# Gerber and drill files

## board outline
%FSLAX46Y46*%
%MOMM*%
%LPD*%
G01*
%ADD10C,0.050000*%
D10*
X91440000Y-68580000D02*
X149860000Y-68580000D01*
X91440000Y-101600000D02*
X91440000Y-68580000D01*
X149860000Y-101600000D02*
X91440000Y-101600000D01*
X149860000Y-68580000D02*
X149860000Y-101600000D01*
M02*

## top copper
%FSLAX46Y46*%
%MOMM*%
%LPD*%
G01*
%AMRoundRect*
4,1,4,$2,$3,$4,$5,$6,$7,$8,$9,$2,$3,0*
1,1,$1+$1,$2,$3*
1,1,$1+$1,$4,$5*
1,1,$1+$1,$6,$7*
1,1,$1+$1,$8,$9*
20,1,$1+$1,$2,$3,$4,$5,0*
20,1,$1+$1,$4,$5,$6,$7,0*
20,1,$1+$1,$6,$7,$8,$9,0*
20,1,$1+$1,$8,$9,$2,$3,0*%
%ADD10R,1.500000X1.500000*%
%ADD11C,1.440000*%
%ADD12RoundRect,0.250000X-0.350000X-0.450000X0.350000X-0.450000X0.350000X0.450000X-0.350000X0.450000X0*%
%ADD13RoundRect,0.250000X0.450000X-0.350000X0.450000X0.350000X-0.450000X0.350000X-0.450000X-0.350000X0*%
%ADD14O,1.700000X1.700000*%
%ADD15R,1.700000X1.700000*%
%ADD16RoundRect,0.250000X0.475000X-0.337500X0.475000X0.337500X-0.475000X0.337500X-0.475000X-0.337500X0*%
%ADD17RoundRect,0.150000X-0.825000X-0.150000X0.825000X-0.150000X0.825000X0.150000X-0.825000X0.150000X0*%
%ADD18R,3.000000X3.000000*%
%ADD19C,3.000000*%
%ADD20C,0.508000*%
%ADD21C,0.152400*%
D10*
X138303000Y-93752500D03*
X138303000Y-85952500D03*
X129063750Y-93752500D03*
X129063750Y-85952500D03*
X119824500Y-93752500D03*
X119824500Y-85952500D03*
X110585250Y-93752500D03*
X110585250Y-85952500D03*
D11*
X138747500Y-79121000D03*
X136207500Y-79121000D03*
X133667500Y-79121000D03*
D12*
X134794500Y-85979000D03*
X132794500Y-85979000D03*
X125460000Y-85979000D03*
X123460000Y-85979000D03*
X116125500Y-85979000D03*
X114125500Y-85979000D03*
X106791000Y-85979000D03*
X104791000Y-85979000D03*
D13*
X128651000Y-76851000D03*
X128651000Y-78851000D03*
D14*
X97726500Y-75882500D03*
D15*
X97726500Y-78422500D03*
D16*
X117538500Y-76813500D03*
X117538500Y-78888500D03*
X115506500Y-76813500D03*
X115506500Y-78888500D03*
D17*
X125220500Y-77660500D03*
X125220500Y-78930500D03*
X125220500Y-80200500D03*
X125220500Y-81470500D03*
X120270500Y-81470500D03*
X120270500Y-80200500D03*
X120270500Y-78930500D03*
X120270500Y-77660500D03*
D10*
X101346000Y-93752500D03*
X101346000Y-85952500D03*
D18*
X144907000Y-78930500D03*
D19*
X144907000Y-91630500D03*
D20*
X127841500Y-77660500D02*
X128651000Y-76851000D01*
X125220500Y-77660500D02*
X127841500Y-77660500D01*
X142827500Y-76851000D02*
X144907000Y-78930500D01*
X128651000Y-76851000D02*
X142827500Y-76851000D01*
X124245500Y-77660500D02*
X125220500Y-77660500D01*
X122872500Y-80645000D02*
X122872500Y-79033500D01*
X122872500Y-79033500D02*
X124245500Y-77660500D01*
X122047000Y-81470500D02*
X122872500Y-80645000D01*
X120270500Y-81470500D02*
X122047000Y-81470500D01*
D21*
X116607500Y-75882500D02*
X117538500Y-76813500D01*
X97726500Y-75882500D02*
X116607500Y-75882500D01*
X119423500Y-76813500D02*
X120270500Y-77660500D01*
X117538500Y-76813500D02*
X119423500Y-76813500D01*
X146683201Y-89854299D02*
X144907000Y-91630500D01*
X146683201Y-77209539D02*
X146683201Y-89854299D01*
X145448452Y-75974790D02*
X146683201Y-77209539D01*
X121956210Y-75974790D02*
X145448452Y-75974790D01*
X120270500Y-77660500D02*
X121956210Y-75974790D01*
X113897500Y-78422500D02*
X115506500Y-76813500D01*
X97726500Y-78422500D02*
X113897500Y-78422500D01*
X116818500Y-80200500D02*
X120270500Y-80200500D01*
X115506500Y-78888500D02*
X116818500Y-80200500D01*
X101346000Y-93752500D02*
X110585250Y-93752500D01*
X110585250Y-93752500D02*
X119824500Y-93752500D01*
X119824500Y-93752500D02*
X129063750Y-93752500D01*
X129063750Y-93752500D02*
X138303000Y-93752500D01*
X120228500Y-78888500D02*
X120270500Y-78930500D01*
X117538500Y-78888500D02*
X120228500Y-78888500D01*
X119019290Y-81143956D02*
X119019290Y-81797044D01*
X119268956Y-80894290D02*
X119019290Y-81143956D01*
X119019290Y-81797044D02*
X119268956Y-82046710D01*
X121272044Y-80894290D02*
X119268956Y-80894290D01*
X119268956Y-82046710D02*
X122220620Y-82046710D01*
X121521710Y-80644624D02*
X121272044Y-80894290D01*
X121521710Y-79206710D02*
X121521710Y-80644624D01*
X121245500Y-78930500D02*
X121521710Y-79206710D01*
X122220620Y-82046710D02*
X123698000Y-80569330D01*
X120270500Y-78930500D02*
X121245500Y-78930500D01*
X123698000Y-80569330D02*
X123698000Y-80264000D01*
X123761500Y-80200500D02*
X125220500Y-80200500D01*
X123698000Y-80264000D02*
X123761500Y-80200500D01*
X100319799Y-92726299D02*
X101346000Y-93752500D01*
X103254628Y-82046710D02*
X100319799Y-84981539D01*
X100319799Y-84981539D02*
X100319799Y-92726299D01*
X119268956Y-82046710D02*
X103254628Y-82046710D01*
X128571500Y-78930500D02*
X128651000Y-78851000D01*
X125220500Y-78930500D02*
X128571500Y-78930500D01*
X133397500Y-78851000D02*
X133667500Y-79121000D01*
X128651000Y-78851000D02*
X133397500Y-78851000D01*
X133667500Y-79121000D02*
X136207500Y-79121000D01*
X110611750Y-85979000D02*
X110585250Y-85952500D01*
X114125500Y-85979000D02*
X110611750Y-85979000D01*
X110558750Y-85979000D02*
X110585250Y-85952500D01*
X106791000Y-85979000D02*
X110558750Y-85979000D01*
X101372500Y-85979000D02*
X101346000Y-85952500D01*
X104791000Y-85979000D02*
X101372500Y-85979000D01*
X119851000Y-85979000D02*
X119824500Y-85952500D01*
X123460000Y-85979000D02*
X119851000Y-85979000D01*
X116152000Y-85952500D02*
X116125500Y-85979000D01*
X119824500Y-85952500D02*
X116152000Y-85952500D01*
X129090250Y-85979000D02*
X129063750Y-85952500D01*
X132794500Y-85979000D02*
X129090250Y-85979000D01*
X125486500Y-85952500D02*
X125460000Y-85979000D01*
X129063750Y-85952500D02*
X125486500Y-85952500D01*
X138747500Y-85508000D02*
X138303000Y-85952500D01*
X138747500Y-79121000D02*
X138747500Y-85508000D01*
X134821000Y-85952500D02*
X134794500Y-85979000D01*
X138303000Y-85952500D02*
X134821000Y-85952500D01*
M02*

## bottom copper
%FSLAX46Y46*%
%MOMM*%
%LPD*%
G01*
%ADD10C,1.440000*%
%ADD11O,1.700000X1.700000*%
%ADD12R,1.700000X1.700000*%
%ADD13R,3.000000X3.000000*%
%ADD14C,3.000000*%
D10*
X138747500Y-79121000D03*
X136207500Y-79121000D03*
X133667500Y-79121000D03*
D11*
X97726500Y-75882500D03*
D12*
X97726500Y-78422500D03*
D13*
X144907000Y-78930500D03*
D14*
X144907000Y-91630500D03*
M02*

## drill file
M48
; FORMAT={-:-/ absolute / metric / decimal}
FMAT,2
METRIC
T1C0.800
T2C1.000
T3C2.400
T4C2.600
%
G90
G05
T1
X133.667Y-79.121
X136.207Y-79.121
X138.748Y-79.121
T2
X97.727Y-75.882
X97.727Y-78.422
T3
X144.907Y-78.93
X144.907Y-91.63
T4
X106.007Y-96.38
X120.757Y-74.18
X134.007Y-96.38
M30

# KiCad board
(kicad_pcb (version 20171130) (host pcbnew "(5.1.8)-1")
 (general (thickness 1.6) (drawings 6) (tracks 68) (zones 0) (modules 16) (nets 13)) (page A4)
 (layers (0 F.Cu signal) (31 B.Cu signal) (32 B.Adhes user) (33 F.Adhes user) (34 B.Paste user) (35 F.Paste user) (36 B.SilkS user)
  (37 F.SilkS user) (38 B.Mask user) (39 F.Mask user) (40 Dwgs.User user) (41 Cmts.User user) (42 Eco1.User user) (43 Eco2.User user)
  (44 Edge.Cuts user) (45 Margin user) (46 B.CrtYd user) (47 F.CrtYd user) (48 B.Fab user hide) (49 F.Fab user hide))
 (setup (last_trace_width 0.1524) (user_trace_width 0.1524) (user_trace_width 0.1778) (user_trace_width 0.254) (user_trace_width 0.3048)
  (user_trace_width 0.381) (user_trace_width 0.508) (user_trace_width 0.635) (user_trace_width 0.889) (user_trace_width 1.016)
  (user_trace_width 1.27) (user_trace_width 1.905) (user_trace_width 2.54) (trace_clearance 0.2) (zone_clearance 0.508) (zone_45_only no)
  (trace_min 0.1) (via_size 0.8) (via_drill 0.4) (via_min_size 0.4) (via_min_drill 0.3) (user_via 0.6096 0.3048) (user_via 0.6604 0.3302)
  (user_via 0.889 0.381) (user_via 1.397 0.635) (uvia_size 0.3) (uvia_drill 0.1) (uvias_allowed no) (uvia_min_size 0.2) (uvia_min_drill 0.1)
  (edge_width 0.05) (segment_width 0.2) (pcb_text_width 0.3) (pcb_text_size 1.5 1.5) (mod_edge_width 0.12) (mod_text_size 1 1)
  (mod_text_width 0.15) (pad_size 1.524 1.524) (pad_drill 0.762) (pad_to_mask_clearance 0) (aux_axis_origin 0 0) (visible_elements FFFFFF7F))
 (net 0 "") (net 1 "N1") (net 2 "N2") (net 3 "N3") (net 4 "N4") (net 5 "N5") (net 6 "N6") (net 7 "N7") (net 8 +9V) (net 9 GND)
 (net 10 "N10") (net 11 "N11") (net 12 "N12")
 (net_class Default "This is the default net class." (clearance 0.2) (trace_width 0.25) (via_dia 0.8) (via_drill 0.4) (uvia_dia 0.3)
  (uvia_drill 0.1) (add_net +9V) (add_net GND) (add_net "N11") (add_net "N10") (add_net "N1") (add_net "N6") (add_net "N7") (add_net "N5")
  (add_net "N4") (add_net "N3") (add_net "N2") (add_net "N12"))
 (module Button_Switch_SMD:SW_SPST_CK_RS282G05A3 (layer F.Cu) (at 138.303 89.8525 270)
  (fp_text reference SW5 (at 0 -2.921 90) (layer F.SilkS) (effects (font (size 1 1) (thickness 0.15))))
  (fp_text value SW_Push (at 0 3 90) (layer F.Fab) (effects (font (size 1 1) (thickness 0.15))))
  (pad 2 smd rect (at 3.9 0 270) (size 1.5 1.5) (layers F.Cu F.Paste F.Mask) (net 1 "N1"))
  (pad 1 smd rect (at -3.9 0 270) (size 1.5 1.5) (layers F.Cu F.Paste F.Mask) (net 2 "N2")))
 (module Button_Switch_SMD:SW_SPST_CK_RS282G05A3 (layer F.Cu) (at 129.06375 89.8525 270)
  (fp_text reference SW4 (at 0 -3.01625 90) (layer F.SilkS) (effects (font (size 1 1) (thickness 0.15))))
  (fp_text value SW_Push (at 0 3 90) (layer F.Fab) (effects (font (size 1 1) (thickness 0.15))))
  (pad 2 smd rect (at 3.9 0 270) (size 1.5 1.5) (layers F.Cu F.Paste F.Mask) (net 1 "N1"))
  (pad 1 smd rect (at -3.9 0 270) (size 1.5 1.5) (layers F.Cu F.Paste F.Mask) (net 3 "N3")))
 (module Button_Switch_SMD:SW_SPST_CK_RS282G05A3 (layer F.Cu) (at 119.8245 89.8525 270)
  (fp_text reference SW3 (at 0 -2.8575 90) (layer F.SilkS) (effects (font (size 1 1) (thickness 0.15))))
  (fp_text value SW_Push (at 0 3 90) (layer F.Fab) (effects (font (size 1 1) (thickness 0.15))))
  (pad 2 smd rect (at 3.9 0 270) (size 1.5 1.5) (layers F.Cu F.Paste F.Mask) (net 1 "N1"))
  (pad 1 smd rect (at -3.9 0 270) (size 1.5 1.5) (layers F.Cu F.Paste F.Mask) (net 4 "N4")))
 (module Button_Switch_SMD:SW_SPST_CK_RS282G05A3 (layer F.Cu) (at 110.58525 89.8525 270)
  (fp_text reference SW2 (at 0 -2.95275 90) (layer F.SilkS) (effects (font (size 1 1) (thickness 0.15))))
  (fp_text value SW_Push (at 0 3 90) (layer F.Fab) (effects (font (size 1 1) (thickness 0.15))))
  (pad 2 smd rect (at 3.9 0 270) (size 1.5 1.5) (layers F.Cu F.Paste F.Mask) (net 1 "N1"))
  (pad 1 smd rect (at -3.9 0 270) (size 1.5 1.5) (layers F.Cu F.Paste F.Mask) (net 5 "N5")))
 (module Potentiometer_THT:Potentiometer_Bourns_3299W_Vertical (layer F.Cu) (at 133.6675 79.121 180)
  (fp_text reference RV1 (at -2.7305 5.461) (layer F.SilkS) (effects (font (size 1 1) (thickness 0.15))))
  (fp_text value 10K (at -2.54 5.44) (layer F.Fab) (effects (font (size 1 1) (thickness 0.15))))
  (pad 3 thru_hole circle (at -5.08 0 180) (size 1.44 1.44) (drill 0.8) (layers *.Cu *.Mask) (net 2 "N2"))
  (pad 2 thru_hole circle (at -2.54 0 180) (size 1.44 1.44) (drill 0.8) (layers *.Cu *.Mask) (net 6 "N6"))
  (pad 1 thru_hole circle (at 0 0 180) (size 1.44 1.44) (drill 0.8) (layers *.Cu *.Mask) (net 6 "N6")))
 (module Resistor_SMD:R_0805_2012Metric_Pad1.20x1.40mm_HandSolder (layer F.Cu) (at 133.7945 85.979)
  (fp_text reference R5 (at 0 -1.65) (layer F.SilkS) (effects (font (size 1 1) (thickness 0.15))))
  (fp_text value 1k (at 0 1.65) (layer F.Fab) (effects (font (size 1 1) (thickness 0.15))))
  (pad 2 smd roundrect (at 1 0) (size 1.2 1.4) (layers F.Cu F.Paste F.Mask) (roundrect_rratio 0.208333) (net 2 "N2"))
  (pad 1 smd roundrect (at -1 0) (size 1.2 1.4) (layers F.Cu F.Paste F.Mask) (roundrect_rratio 0.208333) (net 3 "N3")))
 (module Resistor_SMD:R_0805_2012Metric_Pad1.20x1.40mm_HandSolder (layer F.Cu) (at 124.46 85.979)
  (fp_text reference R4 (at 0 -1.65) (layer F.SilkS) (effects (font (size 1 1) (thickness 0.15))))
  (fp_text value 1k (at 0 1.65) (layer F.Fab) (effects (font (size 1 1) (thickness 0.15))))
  (pad 2 smd roundrect (at 1 0) (size 1.2 1.4) (layers F.Cu F.Paste F.Mask) (roundrect_rratio 0.208333) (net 3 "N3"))
  (pad 1 smd roundrect (at -1 0) (size 1.2 1.4) (layers F.Cu F.Paste F.Mask) (roundrect_rratio 0.208333) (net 4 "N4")))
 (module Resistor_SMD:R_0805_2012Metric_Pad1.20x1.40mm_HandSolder (layer F.Cu) (at 115.1255 85.979)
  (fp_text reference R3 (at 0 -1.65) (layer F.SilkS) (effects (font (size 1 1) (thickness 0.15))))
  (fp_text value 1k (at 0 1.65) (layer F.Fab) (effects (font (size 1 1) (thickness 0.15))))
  (pad 2 smd roundrect (at 1 0) (size 1.2 1.4) (layers F.Cu F.Paste F.Mask) (roundrect_rratio 0.208333) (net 4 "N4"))
  (pad 1 smd roundrect (at -1 0) (size 1.2 1.4) (layers F.Cu F.Paste F.Mask) (roundrect_rratio 0.208333) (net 5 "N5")))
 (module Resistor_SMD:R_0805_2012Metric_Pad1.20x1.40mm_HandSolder (layer F.Cu) (at 105.791 85.979)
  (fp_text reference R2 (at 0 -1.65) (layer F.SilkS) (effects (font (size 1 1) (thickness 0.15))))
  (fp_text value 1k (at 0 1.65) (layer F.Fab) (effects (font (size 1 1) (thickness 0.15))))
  (pad 2 smd roundrect (at 1 0) (size 1.2 1.4) (layers F.Cu F.Paste F.Mask) (roundrect_rratio 0.208333) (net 5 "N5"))
  (pad 1 smd roundrect (at -1 0) (size 1.2 1.4) (layers F.Cu F.Paste F.Mask) (roundrect_rratio 0.208333) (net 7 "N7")))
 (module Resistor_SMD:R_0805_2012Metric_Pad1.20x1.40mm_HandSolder (layer F.Cu) (at 128.651 77.851 90)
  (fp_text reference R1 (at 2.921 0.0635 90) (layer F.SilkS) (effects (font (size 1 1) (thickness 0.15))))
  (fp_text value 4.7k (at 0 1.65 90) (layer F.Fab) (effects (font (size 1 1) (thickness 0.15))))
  (pad 2 smd roundrect (at 1 0 90) (size 1.2 1.4) (layers F.Cu F.Paste F.Mask) (roundrect_rratio 0.208333) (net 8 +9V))
  (pad 1 smd roundrect (at -1 0 90) (size 1.2 1.4) (layers F.Cu F.Paste F.Mask) (roundrect_rratio 0.208333) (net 6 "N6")))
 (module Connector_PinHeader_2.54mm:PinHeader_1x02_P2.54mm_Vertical (layer F.Cu) (at 97.7265 78.4225 180)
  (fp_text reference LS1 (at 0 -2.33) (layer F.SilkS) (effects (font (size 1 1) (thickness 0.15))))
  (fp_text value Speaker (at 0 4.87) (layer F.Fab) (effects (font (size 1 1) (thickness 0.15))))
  (pad 2 thru_hole oval (at 0 2.54 180) (size 1.7 1.7) (drill 1) (layers *.Cu *.Mask) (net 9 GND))
  (pad 1 thru_hole rect (at 0 0 180) (size 1.7 1.7) (drill 1) (layers *.Cu *.Mask) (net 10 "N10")))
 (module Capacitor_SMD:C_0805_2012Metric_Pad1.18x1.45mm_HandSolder (layer F.Cu) (at 117.5385 77.851 90)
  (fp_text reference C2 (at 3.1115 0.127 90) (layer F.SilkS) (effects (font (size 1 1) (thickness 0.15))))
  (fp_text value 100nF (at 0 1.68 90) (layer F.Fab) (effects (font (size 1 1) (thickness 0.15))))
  (pad 2 smd roundrect (at 1.0375 0 90) (size 1.175 1.45) (layers F.Cu F.Paste F.Mask) (roundrect_rratio 0.212766) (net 9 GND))
  (pad 1 smd roundrect (at -1.0375 0 90) (size 1.175 1.45) (layers F.Cu F.Paste F.Mask) (roundrect_rratio 0.212766) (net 1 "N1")))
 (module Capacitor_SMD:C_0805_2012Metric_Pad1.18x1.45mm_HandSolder (layer F.Cu) (at 115.5065 77.851 90)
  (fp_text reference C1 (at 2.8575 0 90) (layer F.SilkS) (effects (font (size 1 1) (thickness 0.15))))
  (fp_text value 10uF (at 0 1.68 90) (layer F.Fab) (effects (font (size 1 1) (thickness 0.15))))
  (pad 2 smd roundrect (at 1.0375 0 90) (size 1.175 1.45) (layers F.Cu F.Paste F.Mask) (roundrect_rratio 0.212766) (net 10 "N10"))
  (pad 1 smd roundrect (at -1.0375 0 90) (size 1.175 1.45) (layers F.Cu F.Paste F.Mask) (roundrect_rratio 0.212766) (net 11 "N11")))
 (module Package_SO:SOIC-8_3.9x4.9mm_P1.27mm (layer F.Cu) (at 122.7455 79.5655)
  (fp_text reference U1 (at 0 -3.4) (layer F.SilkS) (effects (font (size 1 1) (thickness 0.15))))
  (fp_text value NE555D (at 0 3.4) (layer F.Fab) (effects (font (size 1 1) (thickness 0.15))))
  (pad 8 smd roundrect (at 2.475 -1.905) (size 1.95 0.6) (layers F.Cu F.Paste F.Mask) (roundrect_rratio 0.25) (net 8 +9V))
  (pad 7 smd roundrect (at 2.475 -0.635) (size 1.95 0.6) (layers F.Cu F.Paste F.Mask) (roundrect_rratio 0.25) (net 6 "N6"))
  (pad 6 smd roundrect (at 2.475 0.635) (size 1.95 0.6) (layers F.Cu F.Paste F.Mask) (roundrect_rratio 0.25) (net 1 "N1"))
  (pad 5 smd roundrect (at 2.475 1.905) (size 1.95 0.6) (layers F.Cu F.Paste F.Mask) (roundrect_rratio 0.25) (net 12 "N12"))
  (pad 4 smd roundrect (at -2.475 1.905) (size 1.95 0.6) (layers F.Cu F.Paste F.Mask) (roundrect_rratio 0.25) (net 8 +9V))
  (pad 3 smd roundrect (at -2.475 0.635) (size 1.95 0.6) (layers F.Cu F.Paste F.Mask) (roundrect_rratio 0.25) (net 11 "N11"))
  (pad 2 smd roundrect (at -2.475 -0.635) (size 1.95 0.6) (layers F.Cu F.Paste F.Mask) (roundrect_rratio 0.25) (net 1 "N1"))
  (pad 1 smd roundrect (at -2.475 -1.905) (size 1.95 0.6) (layers F.Cu F.Paste F.Mask) (roundrect_rratio 0.25) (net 9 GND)))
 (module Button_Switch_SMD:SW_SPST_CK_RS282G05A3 (layer F.Cu) (at 101.346 89.8525 270)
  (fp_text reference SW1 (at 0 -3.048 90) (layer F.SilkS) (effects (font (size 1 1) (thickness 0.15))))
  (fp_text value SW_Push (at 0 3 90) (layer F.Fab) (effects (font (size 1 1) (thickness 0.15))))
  (pad 2 smd rect (at 3.9 0 270) (size 1.5 1.5) (layers F.Cu F.Paste F.Mask) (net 1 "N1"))
  (pad 1 smd rect (at -3.9 0 270) (size 1.5 1.5) (layers F.Cu F.Paste F.Mask) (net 7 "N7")))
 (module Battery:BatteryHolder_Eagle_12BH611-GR (layer B.Cu) (at 144.907 78.9305)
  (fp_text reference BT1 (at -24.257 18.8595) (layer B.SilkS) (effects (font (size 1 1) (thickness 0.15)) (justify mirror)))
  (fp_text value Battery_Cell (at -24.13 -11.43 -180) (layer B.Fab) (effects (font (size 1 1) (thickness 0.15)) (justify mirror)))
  (pad "" np_thru_hole circle (at -24.15 -4.75) (size 2.6 2.6) (drill 2.6) (layers *.Cu *.Mask))
  (pad "" np_thru_hole circle (at -38.9 17.45) (size 2.6 2.6) (drill 2.6) (layers *.Cu *.Mask))
  (pad "" np_thru_hole circle (at -10.9 17.45) (size 2.6 2.6) (drill 2.6) (layers *.Cu *.Mask))
  (pad 1 thru_hole rect (at 0 0) (size 3 3) (drill 2.4) (layers *.Cu *.Mask) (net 8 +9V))
  (pad 2 thru_hole circle (at 0 12.7) (size 3 3) (drill 2.4) (layers *.Cu *.Mask) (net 9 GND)))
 (gr_line (start 91.44 68.58) (end 149.86 68.58) (layer Edge.Cuts) (width 0.05))
 (gr_line (start 91.44 101.6) (end 91.44 68.58) (layer Edge.Cuts) (width 0.05))
 (gr_line (start 149.86 101.6) (end 91.44 101.6) (layer Edge.Cuts) (width 0.05))
 (gr_line (start 149.86 68.58) (end 149.86 101.6) (layer Edge.Cuts) (width 0.05))
 (segment (start 127.8415 77.6605) (end 128.651 76.851) (width 0.508) (layer F.Cu) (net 8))
 (segment (start 125.2205 77.6605) (end 127.8415 77.6605) (width 0.508) (layer F.Cu) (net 8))
 (segment (start 142.8275 76.851) (end 144.907 78.9305) (width 0.508) (layer F.Cu) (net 8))
 (segment (start 128.651 76.851) (end 142.8275 76.851) (width 0.508) (layer F.Cu) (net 8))
 (segment (start 124.2455 77.6605) (end 125.2205 77.6605) (width 0.508) (layer F.Cu) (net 8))
 (segment (start 122.8725 80.645) (end 122.8725 79.0335) (width 0.508) (layer F.Cu) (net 8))
 (segment (start 122.8725 79.0335) (end 124.2455 77.6605) (width 0.508) (layer F.Cu) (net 8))
 (segment (start 122.047 81.4705) (end 122.8725 80.645) (width 0.508) (layer F.Cu) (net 8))
 (segment (start 120.2705 81.4705) (end 122.047 81.4705) (width 0.508) (layer F.Cu) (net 8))
 (segment (start 116.6075 75.8825) (end 117.5385 76.8135) (width 0.1524) (layer F.Cu) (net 9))
 (segment (start 97.7265 75.8825) (end 116.6075 75.8825) (width 0.1524) (layer F.Cu) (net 9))
 (segment (start 119.4235 76.8135) (end 120.2705 77.6605) (width 0.1524) (layer F.Cu) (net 9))
 (segment (start 117.5385 76.8135) (end 119.4235 76.8135) (width 0.1524) (layer F.Cu) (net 9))
 (segment (start 146.683201 89.854299) (end 144.907 91.6305) (width 0.1524) (layer F.Cu) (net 9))
 (segment (start 146.683201 77.209539) (end 146.683201 89.854299) (width 0.1524) (layer F.Cu) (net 9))
 (segment (start 145.448452 75.97479) (end 146.683201 77.209539) (width 0.1524) (layer F.Cu) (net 9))
 (segment (start 121.95621 75.97479) (end 145.448452 75.97479) (width 0.1524) (layer F.Cu) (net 9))
 (segment (start 120.2705 77.6605) (end 121.95621 75.97479) (width 0.1524) (layer F.Cu) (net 9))
 (segment (start 113.8975 78.4225) (end 115.5065 76.8135) (width 0.1524) (layer F.Cu) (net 10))
 (segment (start 97.7265 78.4225) (end 113.8975 78.4225) (width 0.1524) (layer F.Cu) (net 10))
 (segment (start 116.8185 80.2005) (end 120.2705 80.2005) (width 0.1524) (layer F.Cu) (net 11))
 (segment (start 115.5065 78.8885) (end 116.8185 80.2005) (width 0.1524) (layer F.Cu) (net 11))
 (segment (start 101.346 93.7525) (end 110.58525 93.7525) (width 0.1524) (layer F.Cu) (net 1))
 (segment (start 110.58525 93.7525) (end 119.8245 93.7525) (width 0.1524) (layer F.Cu) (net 1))
 (segment (start 119.8245 93.7525) (end 129.06375 93.7525) (width 0.1524) (layer F.Cu) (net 1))
 (segment (start 129.06375 93.7525) (end 138.303 93.7525) (width 0.1524) (layer F.Cu) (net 1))
 (segment (start 120.2285 78.8885) (end 120.2705 78.9305) (width 0.1524) (layer F.Cu) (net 1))
 (segment (start 117.5385 78.8885) (end 120.2285 78.8885) (width 0.1524) (layer F.Cu) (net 1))
 (segment (start 119.01929 81.143956) (end 119.01929 81.797044) (width 0.1524) (layer F.Cu) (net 1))
 (segment (start 119.268956 80.89429) (end 119.01929 81.143956) (width 0.1524) (layer F.Cu) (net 1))
 (segment (start 119.01929 81.797044) (end 119.268956 82.04671) (width 0.1524) (layer F.Cu) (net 1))
 (segment (start 121.272044 80.89429) (end 119.268956 80.89429) (width 0.1524) (layer F.Cu) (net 1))
 (segment (start 119.268956 82.04671) (end 122.22062 82.04671) (width 0.1524) (layer F.Cu) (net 1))
 (segment (start 121.52171 80.644624) (end 121.272044 80.89429) (width 0.1524) (layer F.Cu) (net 1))
 (segment (start 121.52171 79.20671) (end 121.52171 80.644624) (width 0.1524) (layer F.Cu) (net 1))
 (segment (start 121.2455 78.9305) (end 121.52171 79.20671) (width 0.1524) (layer F.Cu) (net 1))
 (segment (start 122.22062 82.04671) (end 123.698 80.56933) (width 0.1524) (layer F.Cu) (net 1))
 (segment (start 120.2705 78.9305) (end 121.2455 78.9305) (width 0.1524) (layer F.Cu) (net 1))
 (segment (start 123.698 80.56933) (end 123.698 80.264) (width 0.1524) (layer F.Cu) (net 1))
 (segment (start 123.7615 80.2005) (end 125.2205 80.2005) (width 0.1524) (layer F.Cu) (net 1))
 (segment (start 123.698 80.264) (end 123.7615 80.2005) (width 0.1524) (layer F.Cu) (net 1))
 (segment (start 100.319799 92.726299) (end 101.346 93.7525) (width 0.1524) (layer F.Cu) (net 1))
 (segment (start 103.254628 82.04671) (end 100.319799 84.981539) (width 0.1524) (layer F.Cu) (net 1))
 (segment (start 100.319799 84.981539) (end 100.319799 92.726299) (width 0.1524) (layer F.Cu) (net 1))
 (segment (start 119.268956 82.04671) (end 103.254628 82.04671) (width 0.1524) (layer F.Cu) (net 1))
 (segment (start 128.5715 78.9305) (end 128.651 78.851) (width 0.1524) (layer F.Cu) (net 6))
 (segment (start 125.2205 78.9305) (end 128.5715 78.9305) (width 0.1524) (layer F.Cu) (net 6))
 (segment (start 133.3975 78.851) (end 133.6675 79.121) (width 0.1524) (layer F.Cu) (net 6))
 (segment (start 128.651 78.851) (end 133.3975 78.851) (width 0.1524) (layer F.Cu) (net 6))
 (segment (start 133.6675 79.121) (end 136.2075 79.121) (width 0.1524) (layer F.Cu) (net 6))
 (segment (start 110.61175 85.979) (end 110.58525 85.9525) (width 0.1524) (layer F.Cu) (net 5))
 (segment (start 114.1255 85.979) (end 110.61175 85.979) (width 0.1524) (layer F.Cu) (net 5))
 (segment (start 110.55875 85.979) (end 110.58525 85.9525) (width 0.1524) (layer F.Cu) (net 5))
 (segment (start 106.791 85.979) (end 110.55875 85.979) (width 0.1524) (layer F.Cu) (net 5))
 (segment (start 101.3725 85.979) (end 101.346 85.9525) (width 0.1524) (layer F.Cu) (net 7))
 (segment (start 104.791 85.979) (end 101.3725 85.979) (width 0.1524) (layer F.Cu) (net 7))
 (segment (start 119.851 85.979) (end 119.8245 85.9525) (width 0.1524) (layer F.Cu) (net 4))
 (segment (start 123.46 85.979) (end 119.851 85.979) (width 0.1524) (layer F.Cu) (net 4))
 (segment (start 116.152 85.9525) (end 116.1255 85.979) (width 0.1524) (layer F.Cu) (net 4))
 (segment (start 119.8245 85.9525) (end 116.152 85.9525) (width 0.1524) (layer F.Cu) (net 4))
 (segment (start 129.09025 85.979) (end 129.06375 85.9525) (width 0.1524) (layer F.Cu) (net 3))
 (segment (start 132.7945 85.979) (end 129.09025 85.979) (width 0.1524) (layer F.Cu) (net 3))
 (segment (start 125.4865 85.9525) (end 125.46 85.979) (width 0.1524) (layer F.Cu) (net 3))
 (segment (start 129.06375 85.9525) (end 125.4865 85.9525) (width 0.1524) (layer F.Cu) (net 3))
 (segment (start 138.7475 85.508) (end 138.303 85.9525) (width 0.1524) (layer F.Cu) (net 2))
 (segment (start 138.7475 79.121) (end 138.7475 85.508) (width 0.1524) (layer F.Cu) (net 2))
 (segment (start 134.821 85.9525) (end 134.7945 85.979) (width 0.1524) (layer F.Cu) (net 2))
 (segment (start 138.303 85.9525) (end 134.821 85.9525) (width 0.1524) (layer F.Cu) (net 2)))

